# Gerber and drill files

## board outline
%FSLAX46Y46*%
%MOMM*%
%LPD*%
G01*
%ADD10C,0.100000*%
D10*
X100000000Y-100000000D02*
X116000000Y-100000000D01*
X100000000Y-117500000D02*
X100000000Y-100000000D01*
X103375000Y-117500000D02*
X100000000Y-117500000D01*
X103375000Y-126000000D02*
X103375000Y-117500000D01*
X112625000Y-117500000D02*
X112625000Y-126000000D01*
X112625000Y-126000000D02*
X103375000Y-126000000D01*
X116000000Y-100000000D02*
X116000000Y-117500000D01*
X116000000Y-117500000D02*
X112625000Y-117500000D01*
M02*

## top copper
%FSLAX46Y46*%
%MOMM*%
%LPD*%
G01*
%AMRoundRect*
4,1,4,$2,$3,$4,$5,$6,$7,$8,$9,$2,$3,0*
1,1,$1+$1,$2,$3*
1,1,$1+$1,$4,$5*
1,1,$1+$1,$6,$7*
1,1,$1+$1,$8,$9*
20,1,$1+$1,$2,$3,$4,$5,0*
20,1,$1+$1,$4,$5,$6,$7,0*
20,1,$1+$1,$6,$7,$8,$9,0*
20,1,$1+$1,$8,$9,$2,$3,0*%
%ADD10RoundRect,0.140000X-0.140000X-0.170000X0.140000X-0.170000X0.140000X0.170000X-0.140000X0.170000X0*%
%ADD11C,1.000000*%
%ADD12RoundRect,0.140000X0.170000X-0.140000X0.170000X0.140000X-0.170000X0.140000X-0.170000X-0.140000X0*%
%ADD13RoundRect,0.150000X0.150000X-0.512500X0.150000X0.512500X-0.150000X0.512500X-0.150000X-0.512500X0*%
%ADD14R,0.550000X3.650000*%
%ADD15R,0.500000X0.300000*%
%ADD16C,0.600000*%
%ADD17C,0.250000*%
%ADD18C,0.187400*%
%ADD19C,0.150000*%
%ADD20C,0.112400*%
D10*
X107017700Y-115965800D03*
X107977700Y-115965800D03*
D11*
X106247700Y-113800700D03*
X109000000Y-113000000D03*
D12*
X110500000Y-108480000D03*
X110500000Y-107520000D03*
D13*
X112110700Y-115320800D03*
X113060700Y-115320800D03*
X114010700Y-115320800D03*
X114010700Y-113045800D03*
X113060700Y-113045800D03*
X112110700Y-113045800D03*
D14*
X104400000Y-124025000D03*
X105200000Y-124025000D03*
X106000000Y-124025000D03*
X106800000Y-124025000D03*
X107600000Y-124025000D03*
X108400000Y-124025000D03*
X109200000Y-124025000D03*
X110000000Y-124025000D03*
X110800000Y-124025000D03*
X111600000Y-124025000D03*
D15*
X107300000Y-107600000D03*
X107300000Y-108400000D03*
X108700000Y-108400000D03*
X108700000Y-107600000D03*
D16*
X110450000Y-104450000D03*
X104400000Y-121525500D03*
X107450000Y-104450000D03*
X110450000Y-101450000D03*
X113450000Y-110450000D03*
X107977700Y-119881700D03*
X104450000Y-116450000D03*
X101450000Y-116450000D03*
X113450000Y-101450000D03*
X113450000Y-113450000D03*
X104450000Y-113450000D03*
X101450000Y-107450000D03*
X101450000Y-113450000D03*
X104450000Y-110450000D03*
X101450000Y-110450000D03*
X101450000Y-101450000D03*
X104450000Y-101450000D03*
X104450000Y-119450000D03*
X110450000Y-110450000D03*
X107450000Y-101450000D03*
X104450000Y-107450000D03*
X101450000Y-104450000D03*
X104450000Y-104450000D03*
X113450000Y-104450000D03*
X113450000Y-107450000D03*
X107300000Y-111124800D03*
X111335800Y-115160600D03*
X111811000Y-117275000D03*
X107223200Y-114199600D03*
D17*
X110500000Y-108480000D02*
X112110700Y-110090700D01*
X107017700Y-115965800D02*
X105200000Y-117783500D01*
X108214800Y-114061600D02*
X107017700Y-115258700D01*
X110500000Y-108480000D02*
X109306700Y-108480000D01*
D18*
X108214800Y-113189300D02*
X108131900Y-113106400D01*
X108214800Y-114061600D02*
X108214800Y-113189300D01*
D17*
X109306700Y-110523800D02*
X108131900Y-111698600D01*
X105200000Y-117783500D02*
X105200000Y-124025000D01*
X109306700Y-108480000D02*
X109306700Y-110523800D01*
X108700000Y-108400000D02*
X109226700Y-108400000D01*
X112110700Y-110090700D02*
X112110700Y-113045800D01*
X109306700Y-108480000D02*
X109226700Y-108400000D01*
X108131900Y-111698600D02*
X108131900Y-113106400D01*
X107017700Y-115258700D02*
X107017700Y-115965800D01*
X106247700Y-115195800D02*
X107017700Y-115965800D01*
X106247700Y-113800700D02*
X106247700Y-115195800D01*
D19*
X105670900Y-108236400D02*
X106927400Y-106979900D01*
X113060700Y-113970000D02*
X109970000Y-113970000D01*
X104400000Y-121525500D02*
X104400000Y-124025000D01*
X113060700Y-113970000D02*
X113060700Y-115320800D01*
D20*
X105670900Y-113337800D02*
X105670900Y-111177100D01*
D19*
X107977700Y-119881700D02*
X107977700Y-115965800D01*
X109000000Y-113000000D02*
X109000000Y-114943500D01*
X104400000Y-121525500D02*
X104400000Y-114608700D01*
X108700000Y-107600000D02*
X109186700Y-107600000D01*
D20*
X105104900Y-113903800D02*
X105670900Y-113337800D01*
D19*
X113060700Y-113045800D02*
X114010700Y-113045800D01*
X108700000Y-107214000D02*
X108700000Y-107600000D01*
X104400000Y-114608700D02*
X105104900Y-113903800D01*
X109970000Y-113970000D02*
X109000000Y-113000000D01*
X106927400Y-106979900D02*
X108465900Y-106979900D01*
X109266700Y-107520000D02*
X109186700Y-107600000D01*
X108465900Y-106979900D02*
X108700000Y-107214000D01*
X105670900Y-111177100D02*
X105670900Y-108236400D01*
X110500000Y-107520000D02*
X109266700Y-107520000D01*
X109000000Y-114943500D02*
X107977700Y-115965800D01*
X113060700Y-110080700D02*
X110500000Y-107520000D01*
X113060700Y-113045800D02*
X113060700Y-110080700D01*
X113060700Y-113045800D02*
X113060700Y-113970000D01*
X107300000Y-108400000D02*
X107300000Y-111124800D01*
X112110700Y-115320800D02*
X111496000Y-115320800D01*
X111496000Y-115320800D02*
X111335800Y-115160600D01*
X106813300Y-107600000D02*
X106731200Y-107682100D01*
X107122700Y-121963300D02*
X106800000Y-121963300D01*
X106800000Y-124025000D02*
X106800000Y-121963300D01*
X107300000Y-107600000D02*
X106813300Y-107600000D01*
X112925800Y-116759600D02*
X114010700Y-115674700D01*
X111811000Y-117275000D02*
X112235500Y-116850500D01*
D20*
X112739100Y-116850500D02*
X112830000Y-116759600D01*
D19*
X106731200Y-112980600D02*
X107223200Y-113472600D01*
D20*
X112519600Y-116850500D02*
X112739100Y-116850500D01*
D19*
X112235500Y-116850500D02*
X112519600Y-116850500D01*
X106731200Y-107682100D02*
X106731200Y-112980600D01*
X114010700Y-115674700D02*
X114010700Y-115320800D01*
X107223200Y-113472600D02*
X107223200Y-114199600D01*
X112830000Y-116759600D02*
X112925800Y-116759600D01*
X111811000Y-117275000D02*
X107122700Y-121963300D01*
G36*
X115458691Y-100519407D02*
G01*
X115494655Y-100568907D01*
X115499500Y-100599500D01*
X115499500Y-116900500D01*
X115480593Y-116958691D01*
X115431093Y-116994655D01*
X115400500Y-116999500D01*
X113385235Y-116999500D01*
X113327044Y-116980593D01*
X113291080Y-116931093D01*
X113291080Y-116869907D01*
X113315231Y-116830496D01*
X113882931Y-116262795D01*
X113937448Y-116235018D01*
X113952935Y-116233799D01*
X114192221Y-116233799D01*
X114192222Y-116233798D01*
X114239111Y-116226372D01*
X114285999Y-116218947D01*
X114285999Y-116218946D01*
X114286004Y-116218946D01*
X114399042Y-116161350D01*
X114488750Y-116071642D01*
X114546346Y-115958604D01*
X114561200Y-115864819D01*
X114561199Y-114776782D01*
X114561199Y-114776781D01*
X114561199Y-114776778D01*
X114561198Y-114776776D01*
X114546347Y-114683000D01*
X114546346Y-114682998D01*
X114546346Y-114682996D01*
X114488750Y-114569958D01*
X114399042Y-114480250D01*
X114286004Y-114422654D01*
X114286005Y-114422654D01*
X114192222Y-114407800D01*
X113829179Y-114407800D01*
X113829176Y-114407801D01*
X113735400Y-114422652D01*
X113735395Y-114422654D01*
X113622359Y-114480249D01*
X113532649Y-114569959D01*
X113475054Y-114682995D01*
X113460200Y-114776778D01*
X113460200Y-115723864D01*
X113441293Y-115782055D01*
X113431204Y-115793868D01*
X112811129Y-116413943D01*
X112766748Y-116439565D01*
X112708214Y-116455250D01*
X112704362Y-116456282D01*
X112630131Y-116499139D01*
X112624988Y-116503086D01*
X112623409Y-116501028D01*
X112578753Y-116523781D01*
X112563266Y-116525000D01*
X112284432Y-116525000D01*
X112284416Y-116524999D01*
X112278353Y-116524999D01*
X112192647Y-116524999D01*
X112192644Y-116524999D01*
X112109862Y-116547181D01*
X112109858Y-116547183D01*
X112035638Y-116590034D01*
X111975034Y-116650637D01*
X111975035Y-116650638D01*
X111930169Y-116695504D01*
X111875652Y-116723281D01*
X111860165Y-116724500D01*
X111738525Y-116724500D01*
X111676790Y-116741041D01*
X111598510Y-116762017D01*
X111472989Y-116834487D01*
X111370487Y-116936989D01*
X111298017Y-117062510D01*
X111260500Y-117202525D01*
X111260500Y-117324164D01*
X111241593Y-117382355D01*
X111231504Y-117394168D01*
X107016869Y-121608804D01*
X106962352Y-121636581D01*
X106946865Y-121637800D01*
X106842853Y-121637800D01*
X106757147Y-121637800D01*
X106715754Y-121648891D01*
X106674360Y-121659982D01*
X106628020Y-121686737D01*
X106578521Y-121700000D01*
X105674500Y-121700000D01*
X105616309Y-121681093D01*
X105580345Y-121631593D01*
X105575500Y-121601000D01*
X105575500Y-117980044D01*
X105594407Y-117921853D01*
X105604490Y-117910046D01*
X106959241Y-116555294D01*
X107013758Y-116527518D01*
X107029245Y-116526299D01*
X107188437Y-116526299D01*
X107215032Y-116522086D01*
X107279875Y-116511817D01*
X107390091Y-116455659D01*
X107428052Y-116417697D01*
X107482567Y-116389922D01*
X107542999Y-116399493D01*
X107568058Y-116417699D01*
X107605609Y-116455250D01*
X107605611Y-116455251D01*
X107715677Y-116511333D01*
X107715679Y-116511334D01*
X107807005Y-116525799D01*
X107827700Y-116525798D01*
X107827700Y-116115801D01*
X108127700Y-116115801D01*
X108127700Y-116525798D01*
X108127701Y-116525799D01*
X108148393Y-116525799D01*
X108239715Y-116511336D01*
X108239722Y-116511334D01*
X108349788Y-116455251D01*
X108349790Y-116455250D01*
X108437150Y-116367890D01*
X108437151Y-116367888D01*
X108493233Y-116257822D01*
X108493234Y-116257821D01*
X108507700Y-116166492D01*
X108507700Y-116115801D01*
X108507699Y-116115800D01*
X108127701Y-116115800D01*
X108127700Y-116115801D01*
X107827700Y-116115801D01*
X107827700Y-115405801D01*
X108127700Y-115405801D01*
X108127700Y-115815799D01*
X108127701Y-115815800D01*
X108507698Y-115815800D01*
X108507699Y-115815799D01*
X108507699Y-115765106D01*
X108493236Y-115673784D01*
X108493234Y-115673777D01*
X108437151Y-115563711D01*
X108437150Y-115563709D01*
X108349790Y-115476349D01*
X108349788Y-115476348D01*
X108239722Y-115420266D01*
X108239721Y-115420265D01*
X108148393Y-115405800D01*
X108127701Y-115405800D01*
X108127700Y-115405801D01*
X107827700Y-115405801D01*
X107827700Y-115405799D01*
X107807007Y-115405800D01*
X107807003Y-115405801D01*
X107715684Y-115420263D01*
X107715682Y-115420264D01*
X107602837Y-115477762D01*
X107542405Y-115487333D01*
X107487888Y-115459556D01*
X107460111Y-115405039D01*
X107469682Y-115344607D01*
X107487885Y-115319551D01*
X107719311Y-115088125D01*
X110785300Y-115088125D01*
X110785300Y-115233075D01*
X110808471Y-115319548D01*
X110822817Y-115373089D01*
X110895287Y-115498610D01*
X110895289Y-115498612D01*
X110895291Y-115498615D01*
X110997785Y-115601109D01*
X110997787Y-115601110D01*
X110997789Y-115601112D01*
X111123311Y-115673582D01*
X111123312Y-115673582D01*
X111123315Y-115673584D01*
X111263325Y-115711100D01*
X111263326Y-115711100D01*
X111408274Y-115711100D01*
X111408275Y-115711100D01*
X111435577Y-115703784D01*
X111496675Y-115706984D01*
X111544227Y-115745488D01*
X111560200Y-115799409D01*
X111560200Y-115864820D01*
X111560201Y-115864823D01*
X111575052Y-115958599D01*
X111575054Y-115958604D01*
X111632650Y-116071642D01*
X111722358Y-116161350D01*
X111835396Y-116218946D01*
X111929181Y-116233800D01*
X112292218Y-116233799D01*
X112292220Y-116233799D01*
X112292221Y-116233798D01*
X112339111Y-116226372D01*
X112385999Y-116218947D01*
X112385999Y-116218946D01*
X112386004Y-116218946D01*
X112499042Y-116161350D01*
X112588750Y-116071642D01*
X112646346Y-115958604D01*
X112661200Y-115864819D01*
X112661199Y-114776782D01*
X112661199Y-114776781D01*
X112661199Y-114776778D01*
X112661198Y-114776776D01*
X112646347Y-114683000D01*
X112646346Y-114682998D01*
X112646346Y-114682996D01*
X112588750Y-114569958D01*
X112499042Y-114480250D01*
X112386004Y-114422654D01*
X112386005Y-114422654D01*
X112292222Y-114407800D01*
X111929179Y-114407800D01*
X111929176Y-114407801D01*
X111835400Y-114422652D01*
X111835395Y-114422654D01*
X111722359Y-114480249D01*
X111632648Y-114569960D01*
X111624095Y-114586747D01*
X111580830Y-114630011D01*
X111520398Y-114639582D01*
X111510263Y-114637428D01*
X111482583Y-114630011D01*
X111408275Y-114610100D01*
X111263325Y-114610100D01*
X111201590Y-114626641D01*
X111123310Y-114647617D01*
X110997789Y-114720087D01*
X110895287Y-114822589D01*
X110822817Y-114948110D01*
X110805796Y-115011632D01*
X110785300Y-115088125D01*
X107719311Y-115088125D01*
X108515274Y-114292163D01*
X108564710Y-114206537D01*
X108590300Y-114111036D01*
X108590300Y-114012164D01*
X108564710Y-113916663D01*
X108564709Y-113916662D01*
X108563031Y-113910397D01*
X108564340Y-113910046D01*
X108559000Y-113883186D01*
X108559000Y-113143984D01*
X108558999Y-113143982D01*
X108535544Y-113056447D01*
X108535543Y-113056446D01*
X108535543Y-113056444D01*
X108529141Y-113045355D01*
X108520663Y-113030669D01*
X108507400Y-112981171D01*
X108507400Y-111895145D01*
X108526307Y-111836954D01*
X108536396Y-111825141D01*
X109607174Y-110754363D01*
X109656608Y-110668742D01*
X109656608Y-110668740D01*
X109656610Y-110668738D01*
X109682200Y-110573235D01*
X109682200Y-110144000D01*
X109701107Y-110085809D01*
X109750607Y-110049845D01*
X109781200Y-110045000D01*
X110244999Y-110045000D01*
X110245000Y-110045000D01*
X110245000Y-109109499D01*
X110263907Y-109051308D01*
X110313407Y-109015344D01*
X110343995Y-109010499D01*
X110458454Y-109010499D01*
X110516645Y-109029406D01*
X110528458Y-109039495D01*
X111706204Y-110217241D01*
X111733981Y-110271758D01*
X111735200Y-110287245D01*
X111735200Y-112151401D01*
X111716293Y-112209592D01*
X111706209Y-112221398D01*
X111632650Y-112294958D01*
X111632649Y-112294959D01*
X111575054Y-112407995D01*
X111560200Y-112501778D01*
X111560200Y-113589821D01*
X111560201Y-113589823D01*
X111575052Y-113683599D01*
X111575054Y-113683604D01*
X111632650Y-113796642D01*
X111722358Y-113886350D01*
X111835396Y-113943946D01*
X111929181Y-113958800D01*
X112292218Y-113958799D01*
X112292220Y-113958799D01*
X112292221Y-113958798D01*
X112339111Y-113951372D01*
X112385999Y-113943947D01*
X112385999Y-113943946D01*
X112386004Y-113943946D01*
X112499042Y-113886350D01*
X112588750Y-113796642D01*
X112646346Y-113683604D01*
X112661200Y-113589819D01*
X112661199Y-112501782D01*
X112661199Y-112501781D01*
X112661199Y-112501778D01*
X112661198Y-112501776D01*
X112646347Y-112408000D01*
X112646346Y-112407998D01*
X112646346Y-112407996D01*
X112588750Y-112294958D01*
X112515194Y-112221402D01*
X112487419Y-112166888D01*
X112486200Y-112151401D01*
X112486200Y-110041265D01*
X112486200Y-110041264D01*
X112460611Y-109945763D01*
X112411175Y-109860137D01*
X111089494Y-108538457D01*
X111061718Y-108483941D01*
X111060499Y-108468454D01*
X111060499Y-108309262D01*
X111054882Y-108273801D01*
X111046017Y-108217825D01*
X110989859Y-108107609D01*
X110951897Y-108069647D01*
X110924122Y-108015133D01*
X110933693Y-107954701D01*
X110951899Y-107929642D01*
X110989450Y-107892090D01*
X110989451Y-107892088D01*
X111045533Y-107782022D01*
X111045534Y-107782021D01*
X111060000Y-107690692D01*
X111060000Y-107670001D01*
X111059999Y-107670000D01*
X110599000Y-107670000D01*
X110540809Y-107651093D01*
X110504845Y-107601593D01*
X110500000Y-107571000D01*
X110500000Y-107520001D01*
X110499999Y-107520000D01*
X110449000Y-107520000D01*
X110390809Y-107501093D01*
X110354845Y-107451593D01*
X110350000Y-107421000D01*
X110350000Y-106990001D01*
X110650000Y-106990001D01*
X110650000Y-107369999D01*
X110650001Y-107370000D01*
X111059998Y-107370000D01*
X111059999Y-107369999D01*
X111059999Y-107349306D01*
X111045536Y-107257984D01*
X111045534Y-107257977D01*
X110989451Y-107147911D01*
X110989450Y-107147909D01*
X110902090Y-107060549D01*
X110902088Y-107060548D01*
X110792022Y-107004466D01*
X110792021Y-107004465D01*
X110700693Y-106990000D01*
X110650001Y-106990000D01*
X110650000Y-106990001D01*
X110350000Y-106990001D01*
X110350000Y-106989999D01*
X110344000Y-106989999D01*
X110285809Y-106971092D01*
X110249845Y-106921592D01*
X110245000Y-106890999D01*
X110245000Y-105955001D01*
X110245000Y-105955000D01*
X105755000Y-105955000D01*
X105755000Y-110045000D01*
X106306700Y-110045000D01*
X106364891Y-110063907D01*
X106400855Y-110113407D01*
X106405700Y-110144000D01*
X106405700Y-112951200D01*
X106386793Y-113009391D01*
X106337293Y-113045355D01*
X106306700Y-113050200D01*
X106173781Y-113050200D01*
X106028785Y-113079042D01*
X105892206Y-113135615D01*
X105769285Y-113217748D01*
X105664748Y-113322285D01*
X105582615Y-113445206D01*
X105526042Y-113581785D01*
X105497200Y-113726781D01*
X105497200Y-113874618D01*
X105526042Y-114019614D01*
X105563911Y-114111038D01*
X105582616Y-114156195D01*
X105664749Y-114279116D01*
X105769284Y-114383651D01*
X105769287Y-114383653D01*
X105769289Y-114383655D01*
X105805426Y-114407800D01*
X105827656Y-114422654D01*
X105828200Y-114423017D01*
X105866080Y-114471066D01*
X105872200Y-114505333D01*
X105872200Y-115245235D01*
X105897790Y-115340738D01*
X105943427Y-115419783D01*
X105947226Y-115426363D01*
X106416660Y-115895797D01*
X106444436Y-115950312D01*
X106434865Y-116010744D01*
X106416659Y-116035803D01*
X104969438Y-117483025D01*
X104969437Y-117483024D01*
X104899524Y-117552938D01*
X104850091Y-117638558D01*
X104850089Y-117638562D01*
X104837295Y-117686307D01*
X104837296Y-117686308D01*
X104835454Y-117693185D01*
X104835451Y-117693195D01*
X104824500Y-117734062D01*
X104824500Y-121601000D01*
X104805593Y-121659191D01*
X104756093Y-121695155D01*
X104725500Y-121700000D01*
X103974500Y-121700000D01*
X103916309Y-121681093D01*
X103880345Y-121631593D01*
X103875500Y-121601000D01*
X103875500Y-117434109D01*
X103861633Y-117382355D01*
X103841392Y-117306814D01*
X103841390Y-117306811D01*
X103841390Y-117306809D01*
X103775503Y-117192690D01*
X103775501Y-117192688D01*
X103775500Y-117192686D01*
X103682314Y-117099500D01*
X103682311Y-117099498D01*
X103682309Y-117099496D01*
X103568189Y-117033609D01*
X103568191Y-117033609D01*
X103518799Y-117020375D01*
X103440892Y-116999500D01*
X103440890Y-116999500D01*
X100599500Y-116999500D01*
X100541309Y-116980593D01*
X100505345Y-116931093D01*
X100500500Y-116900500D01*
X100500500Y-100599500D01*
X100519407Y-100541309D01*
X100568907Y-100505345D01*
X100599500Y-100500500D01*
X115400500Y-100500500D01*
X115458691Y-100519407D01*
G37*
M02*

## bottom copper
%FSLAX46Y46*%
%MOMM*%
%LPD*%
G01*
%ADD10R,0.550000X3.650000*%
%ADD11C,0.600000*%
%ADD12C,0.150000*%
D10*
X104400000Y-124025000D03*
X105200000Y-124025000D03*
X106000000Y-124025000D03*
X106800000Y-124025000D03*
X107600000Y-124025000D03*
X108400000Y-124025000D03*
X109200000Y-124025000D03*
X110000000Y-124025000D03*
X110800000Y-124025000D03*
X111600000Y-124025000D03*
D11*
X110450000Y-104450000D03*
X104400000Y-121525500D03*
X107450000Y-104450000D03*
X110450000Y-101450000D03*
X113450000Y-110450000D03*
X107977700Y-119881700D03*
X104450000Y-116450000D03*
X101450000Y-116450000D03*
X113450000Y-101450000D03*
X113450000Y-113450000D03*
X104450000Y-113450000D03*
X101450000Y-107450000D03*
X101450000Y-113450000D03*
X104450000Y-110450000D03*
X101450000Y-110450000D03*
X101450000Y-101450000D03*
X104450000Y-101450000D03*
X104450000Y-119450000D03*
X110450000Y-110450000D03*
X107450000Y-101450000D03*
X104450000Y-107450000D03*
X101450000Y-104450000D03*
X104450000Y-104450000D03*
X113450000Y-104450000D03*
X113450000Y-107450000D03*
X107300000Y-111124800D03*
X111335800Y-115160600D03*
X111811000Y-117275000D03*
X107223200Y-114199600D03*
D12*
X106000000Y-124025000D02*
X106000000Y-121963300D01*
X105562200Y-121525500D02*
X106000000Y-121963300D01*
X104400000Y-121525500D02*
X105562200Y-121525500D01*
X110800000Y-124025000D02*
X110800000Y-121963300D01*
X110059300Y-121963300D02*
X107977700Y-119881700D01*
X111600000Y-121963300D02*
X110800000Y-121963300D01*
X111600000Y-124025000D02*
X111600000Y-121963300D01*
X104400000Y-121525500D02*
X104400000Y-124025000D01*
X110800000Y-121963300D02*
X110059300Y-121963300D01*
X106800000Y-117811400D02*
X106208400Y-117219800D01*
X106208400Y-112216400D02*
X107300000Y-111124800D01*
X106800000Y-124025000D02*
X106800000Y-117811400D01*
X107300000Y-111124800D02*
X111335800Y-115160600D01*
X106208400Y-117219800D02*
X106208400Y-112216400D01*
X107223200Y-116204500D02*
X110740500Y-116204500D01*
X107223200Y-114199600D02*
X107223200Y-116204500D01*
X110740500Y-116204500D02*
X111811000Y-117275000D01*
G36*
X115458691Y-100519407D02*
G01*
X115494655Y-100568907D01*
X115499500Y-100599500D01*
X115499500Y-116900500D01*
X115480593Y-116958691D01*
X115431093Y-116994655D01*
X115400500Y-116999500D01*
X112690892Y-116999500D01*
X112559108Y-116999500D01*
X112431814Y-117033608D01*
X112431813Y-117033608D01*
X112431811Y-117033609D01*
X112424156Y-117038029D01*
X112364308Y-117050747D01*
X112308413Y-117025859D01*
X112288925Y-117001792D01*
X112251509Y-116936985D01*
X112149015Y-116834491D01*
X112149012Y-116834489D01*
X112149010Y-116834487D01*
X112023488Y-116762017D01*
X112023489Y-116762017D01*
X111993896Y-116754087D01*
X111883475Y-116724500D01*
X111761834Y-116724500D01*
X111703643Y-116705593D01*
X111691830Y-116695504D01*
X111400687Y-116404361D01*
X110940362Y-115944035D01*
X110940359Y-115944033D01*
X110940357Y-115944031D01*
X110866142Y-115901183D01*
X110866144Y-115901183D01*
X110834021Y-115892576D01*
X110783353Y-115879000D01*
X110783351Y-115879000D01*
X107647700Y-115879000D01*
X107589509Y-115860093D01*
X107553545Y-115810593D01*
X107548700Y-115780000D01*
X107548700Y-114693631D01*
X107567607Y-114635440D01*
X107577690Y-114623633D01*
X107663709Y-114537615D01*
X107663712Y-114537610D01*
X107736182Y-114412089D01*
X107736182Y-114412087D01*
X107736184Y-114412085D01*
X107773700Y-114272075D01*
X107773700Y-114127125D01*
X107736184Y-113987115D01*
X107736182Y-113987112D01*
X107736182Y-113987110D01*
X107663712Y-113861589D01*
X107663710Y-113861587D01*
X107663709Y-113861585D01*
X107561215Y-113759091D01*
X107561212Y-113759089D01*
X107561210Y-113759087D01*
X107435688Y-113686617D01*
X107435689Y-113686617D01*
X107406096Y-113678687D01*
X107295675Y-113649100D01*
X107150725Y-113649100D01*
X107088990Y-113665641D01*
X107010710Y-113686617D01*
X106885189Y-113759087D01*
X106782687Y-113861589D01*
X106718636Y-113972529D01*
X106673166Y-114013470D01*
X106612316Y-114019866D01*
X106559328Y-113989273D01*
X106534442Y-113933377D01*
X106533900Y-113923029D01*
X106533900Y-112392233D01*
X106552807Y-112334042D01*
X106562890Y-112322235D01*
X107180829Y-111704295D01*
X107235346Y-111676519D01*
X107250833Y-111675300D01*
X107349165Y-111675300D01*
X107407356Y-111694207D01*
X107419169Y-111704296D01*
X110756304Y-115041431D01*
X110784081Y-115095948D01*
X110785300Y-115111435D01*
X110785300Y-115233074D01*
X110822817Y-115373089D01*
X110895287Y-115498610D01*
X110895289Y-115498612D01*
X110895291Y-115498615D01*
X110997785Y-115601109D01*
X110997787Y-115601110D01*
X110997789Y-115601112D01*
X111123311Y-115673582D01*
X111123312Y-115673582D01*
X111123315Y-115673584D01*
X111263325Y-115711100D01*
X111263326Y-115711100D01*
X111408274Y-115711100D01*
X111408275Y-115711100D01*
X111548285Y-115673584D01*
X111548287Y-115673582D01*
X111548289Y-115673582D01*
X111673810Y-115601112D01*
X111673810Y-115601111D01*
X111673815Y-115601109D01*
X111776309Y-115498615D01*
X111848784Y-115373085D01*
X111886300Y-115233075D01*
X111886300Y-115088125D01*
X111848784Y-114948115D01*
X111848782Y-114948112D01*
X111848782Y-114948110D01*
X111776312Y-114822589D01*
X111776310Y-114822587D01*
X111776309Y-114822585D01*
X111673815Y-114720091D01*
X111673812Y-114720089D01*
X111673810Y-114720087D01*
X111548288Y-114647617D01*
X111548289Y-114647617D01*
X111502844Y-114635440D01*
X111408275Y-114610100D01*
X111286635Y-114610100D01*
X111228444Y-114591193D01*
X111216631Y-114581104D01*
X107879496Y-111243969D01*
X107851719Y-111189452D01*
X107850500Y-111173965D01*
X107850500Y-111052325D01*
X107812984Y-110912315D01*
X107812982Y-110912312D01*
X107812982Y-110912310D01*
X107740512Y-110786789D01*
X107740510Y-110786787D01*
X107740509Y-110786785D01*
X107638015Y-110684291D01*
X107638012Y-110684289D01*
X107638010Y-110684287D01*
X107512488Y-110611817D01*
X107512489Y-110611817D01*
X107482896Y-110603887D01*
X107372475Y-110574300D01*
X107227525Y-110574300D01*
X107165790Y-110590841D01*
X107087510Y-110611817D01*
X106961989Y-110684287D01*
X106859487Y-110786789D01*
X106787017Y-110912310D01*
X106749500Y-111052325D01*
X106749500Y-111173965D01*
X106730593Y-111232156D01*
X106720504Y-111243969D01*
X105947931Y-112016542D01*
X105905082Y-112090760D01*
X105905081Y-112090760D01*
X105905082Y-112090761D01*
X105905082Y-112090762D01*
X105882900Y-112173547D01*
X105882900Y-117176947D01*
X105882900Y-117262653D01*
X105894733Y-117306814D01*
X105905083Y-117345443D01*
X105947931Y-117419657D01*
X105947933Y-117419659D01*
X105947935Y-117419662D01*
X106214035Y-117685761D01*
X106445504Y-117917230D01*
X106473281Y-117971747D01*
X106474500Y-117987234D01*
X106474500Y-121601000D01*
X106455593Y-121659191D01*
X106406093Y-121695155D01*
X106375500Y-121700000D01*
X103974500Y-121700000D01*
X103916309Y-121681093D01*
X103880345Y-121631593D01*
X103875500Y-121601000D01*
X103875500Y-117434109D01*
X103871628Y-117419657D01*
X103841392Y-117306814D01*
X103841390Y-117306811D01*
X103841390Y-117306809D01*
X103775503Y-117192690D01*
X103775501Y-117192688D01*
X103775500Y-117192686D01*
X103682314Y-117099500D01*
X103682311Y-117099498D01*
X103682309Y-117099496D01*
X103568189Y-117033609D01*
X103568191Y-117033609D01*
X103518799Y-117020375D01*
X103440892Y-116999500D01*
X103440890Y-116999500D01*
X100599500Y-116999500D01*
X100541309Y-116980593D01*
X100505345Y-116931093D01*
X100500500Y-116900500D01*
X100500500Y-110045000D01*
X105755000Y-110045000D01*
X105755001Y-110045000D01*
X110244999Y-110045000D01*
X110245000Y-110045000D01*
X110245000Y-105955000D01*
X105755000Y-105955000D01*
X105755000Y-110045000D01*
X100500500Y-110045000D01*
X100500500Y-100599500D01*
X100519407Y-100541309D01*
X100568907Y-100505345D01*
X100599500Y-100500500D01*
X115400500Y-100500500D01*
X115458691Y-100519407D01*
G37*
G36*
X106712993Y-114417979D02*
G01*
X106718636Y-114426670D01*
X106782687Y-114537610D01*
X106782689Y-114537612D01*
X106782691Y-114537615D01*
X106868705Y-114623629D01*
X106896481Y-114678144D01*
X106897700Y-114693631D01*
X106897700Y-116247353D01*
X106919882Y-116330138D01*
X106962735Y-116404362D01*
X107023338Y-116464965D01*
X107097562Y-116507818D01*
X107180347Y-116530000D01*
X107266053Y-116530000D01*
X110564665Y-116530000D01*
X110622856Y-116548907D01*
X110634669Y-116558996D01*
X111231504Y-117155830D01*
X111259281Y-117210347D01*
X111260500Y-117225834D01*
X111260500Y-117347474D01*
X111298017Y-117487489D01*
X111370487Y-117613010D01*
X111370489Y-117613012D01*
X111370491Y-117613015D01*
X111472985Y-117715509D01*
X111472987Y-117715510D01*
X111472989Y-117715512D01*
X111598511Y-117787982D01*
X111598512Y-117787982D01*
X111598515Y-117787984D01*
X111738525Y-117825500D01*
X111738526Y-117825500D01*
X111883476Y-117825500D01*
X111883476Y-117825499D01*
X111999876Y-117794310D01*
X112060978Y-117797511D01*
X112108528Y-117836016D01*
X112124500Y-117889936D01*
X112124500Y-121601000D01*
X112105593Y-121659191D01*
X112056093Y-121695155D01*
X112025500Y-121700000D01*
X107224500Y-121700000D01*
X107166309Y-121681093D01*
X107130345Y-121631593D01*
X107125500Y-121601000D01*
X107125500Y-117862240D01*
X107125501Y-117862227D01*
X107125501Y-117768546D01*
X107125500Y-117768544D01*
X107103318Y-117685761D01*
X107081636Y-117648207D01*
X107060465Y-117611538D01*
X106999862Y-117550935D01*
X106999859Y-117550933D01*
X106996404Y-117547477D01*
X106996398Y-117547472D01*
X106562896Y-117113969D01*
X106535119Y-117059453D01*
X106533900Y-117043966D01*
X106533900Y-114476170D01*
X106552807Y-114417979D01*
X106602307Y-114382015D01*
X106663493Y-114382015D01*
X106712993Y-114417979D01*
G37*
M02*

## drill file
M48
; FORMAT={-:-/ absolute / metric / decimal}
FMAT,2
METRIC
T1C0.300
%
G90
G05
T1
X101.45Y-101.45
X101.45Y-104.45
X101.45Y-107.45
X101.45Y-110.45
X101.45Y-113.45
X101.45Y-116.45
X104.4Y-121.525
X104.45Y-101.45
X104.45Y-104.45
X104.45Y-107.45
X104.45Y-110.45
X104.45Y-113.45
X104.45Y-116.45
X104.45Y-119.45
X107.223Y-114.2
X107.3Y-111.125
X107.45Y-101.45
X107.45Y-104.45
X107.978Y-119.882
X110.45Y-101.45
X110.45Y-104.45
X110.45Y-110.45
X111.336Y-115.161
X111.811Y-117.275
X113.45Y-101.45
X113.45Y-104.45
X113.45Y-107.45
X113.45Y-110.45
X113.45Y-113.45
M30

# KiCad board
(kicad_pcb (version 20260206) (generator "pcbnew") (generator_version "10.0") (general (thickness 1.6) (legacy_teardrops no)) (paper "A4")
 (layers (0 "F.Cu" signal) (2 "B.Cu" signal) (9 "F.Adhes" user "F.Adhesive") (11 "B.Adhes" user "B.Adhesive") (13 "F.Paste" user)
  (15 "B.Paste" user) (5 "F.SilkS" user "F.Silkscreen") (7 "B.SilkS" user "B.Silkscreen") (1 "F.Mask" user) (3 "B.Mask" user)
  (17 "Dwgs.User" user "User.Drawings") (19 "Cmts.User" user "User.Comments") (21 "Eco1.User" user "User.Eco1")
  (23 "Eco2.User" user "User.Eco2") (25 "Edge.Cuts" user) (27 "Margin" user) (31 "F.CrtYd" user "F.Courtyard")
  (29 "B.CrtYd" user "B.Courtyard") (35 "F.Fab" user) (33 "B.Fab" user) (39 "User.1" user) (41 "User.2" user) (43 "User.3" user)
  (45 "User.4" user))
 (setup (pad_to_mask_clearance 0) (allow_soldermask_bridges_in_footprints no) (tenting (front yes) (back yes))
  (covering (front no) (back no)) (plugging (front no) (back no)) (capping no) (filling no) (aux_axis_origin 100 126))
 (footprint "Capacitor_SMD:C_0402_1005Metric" (layer "F.Cu") (at 107.4977 115.9658)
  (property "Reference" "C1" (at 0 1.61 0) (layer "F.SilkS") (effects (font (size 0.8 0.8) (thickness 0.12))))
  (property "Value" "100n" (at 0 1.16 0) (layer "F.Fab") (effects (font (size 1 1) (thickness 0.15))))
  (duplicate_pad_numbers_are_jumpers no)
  (pad "1" smd roundrect (at -0.48 0) (size 0.56 0.62) (layers "F.Cu" "F.Mask" "F.Paste") (roundrect_rratio 0.25) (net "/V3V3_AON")
   (zone_connect 1))
  (pad "2" smd roundrect (at 0.48 0) (size 0.56 0.62) (layers "F.Cu" "F.Mask" "F.Paste") (roundrect_rratio 0.25) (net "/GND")
   (zone_connect 1)))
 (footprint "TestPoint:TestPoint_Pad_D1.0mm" (layer "F.Cu") (at 106.2477 113.8007)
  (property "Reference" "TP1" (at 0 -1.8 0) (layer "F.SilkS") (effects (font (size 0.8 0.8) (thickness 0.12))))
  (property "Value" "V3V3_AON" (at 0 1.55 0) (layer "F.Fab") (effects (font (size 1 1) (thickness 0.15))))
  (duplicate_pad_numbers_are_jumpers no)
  (pad "1" smd circle (at 0 0) (size 1 1) (layers "F.Cu" "F.Mask") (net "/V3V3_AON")))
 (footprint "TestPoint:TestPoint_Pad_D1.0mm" (layer "F.Cu") (at 109 113)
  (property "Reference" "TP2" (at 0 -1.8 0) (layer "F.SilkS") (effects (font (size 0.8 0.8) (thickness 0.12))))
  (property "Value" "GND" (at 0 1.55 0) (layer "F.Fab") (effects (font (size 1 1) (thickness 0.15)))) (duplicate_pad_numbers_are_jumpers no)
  (pad "1" smd circle (at 0 0) (size 1 1) (layers "F.Cu" "F.Mask") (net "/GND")))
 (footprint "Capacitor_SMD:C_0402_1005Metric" (layer "F.Cu") (at 110.5 108 90)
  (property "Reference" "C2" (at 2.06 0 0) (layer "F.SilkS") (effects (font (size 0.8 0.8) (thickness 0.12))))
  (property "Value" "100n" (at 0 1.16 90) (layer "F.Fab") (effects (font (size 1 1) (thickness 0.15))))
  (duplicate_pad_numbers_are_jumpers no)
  (pad "1" smd roundrect (at -0.48 0 90) (size 0.56 0.62) (layers "F.Cu" "F.Mask" "F.Paste") (roundrect_rratio 0.25) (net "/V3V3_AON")
   (zone_connect 1))
  (pad "2" smd roundrect (at 0.48 0 90) (size 0.56 0.62) (layers "F.Cu" "F.Mask" "F.Paste") (roundrect_rratio 0.25) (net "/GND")
   (zone_connect 1)))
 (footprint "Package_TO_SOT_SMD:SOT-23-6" (layer "F.Cu") (at 113.0607 114.1833 90)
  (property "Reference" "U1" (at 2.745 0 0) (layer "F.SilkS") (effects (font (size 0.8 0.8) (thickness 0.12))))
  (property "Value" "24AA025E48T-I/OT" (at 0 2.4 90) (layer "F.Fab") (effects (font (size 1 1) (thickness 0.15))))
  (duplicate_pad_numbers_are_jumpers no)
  (pad "1" smd roundrect (at -1.1375 -0.95 90) (size 1.325 0.6) (layers "F.Cu" "F.Mask" "F.Paste") (roundrect_rratio 0.25) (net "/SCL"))
  (pad "2" smd roundrect (at -1.1375 0 90) (size 1.325 0.6) (layers "F.Cu" "F.Mask" "F.Paste") (roundrect_rratio 0.25) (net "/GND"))
  (pad "3" smd roundrect (at -1.1375 0.95 90) (size 1.325 0.6) (layers "F.Cu" "F.Mask" "F.Paste") (roundrect_rratio 0.25) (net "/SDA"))
  (pad "4" smd roundrect (at 1.1375 0.95 90) (size 1.325 0.6) (layers "F.Cu" "F.Mask" "F.Paste") (roundrect_rratio 0.25) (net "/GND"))
  (pad "5" smd roundrect (at 1.1375 0 90) (size 1.325 0.6) (layers "F.Cu" "F.Mask" "F.Paste") (roundrect_rratio 0.25) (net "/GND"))
  (pad "6" smd roundrect (at 1.1375 -0.95 90) (size 1.325 0.6) (layers "F.Cu" "F.Mask" "F.Paste") (roundrect_rratio 0.25) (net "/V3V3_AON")))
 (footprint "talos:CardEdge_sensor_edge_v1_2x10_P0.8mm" (layer "F.Cu") (at 108 124.35)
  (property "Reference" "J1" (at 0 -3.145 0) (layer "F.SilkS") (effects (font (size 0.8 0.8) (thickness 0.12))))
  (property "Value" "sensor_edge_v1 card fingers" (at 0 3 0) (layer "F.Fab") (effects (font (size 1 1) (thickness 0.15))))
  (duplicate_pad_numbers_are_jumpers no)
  (pad "1" smd rect (at -3.6 -0.325) (size 0.55 3.65) (layers "F.Cu" "F.Mask") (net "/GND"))
  (pad "2" smd rect (at -3.6 -0.325) (size 0.55 3.65) (layers "B.Cu" "B.Mask") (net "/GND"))
  (pad "3" smd rect (at -2.8 -0.325) (size 0.55 3.65) (layers "F.Cu" "F.Mask") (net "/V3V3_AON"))
  (pad "4" smd rect (at -2.8 -0.325) (size 0.55 3.65) (layers "B.Cu" "B.Mask") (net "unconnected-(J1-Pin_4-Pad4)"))
  (pad "5" smd rect (at -2 -0.325) (size 0.55 3.65) (layers "F.Cu" "F.Mask") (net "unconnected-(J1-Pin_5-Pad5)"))
  (pad "6" smd rect (at -2 -0.325) (size 0.55 3.65) (layers "B.Cu" "B.Mask") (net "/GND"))
  (pad "7" smd rect (at -1.2 -0.325) (size 0.55 3.65) (layers "F.Cu" "F.Mask") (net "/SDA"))
  (pad "8" smd rect (at -1.2 -0.325) (size 0.55 3.65) (layers "B.Cu" "B.Mask") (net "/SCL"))
  (pad "9" smd rect (at -0.4 -0.325) (size 0.55 3.65) (layers "F.Cu" "F.Mask") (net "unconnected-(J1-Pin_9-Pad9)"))
  (pad "10" smd rect (at -0.4 -0.325) (size 0.55 3.65) (layers "B.Cu" "B.Mask") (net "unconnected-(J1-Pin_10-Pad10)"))
  (pad "11" smd rect (at 0.4 -0.325) (size 0.55 3.65) (layers "F.Cu" "F.Mask") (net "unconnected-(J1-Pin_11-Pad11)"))
  (pad "12" smd rect (at 0.4 -0.325) (size 0.55 3.65) (layers "B.Cu" "B.Mask") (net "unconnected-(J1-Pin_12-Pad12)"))
  (pad "13" smd rect (at 1.2 -0.325) (size 0.55 3.65) (layers "F.Cu" "F.Mask") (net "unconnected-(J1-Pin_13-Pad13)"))
  (pad "14" smd rect (at 1.2 -0.325) (size 0.55 3.65) (layers "B.Cu" "B.Mask") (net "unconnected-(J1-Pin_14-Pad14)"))
  (pad "15" smd rect (at 2 -0.325) (size 0.55 3.65) (layers "F.Cu" "F.Mask") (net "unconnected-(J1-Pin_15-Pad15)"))
  (pad "16" smd rect (at 2 -0.325) (size 0.55 3.65) (layers "B.Cu" "B.Mask") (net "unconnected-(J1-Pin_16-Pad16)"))
  (pad "17" smd rect (at 2.8 -0.325) (size 0.55 3.65) (layers "F.Cu" "F.Mask") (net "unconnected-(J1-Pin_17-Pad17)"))
  (pad "18" smd rect (at 2.8 -0.325) (size 0.55 3.65) (layers "B.Cu" "B.Mask") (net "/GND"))
  (pad "19" smd rect (at 3.6 -0.325) (size 0.55 3.65) (layers "F.Cu" "F.Mask") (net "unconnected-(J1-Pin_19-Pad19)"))
  (pad "20" smd rect (at 3.6 -0.325) (size 0.55 3.65) (layers "B.Cu" "B.Mask") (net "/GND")))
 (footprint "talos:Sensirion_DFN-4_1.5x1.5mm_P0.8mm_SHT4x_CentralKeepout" (layer "F.Cu") (at 108 108)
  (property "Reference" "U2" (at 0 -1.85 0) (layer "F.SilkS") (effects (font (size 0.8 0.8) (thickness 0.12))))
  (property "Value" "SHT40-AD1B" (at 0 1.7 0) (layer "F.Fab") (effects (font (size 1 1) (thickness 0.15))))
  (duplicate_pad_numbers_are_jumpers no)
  (pad "1" smd rect (at -0.7 -0.4) (size 0.5 0.3) (layers "F.Cu" "F.Mask" "F.Paste") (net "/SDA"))
  (pad "2" smd rect (at -0.7 0.4) (size 0.5 0.3) (layers "F.Cu" "F.Mask" "F.Paste") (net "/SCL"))
  (pad "3" smd rect (at 0.7 0.4) (size 0.5 0.3) (layers "F.Cu" "F.Mask" "F.Paste") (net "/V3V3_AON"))
  (pad "4" smd rect (at 0.7 -0.4) (size 0.5 0.3) (layers "F.Cu" "F.Mask" "F.Paste") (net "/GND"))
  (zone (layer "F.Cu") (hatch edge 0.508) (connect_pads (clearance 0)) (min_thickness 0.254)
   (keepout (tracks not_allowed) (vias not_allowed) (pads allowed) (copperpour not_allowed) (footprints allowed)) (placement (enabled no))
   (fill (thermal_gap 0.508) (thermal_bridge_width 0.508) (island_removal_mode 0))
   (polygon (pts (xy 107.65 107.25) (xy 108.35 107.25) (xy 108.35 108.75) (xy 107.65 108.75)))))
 (gr_line (start 100 100) (end 116 100) (stroke (width 0.1) (type default)) (layer "Edge.Cuts"))
 (gr_line (start 100 117.5) (end 100 100) (stroke (width 0.1) (type default)) (layer "Edge.Cuts"))
 (gr_line (start 103.375 117.5) (end 100 117.5) (stroke (width 0.1) (type default)) (layer "Edge.Cuts"))
 (gr_line (start 103.375 126) (end 103.375 117.5) (stroke (width 0.1) (type default)) (layer "Edge.Cuts"))
 (gr_line (start 112.625 117.5) (end 112.625 126) (stroke (width 0.1) (type default)) (layer "Edge.Cuts"))
 (gr_line (start 112.625 126) (end 103.375 126) (stroke (width 0.1) (type default)) (layer "Edge.Cuts"))
 (gr_line (start 116 100) (end 116 117.5) (stroke (width 0.1) (type default)) (layer "Edge.Cuts"))
 (gr_line (start 116 117.5) (end 112.625 117.5) (stroke (width 0.1) (type default)) (layer "Edge.Cuts"))
 (segment (start 110.5 108.48) (end 112.1107 110.0907) (width 0.25) (layer "F.Cu") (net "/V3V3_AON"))
 (segment (start 107.0177 115.9658) (end 105.2 117.7835) (width 0.25) (layer "F.Cu") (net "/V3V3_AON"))
 (segment (start 108.2148 114.0616) (end 107.0177 115.2587) (width 0.25) (layer "F.Cu") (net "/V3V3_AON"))
 (segment (start 110.5 108.48) (end 109.3067 108.48) (width 0.25) (layer "F.Cu") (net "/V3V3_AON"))
 (segment (start 108.2148 113.1893) (end 108.1319 113.1064) (width 0.1874) (layer "F.Cu") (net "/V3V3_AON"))
 (segment (start 108.2148 114.0616) (end 108.2148 113.1893) (width 0.1874) (layer "F.Cu") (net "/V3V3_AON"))
 (segment (start 109.3067 110.5238) (end 108.1319 111.6986) (width 0.25) (layer "F.Cu") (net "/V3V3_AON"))
 (segment (start 105.2 117.7835) (end 105.2 124.025) (width 0.25) (layer "F.Cu") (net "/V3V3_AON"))
 (segment (start 109.3067 108.48) (end 109.3067 110.5238) (width 0.25) (layer "F.Cu") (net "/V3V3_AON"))
 (segment (start 108.7 108.4) (end 109.2267 108.4) (width 0.25) (layer "F.Cu") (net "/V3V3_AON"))
 (segment (start 112.1107 110.0907) (end 112.1107 113.0458) (width 0.25) (layer "F.Cu") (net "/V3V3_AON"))
 (segment (start 109.3067 108.48) (end 109.2267 108.4) (width 0.25) (layer "F.Cu") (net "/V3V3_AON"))
 (segment (start 108.1319 111.6986) (end 108.1319 113.1064) (width 0.25) (layer "F.Cu") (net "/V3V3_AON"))
 (segment (start 107.0177 115.2587) (end 107.0177 115.9658) (width 0.25) (layer "F.Cu") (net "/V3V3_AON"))
 (segment (start 106.2477 115.1958) (end 107.0177 115.9658) (width 0.25) (layer "F.Cu") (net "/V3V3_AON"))
 (segment (start 106.2477 113.8007) (end 106.2477 115.1958) (width 0.25) (layer "F.Cu") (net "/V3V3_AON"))
 (segment (start 105.6709 108.2364) (end 106.9274 106.9799) (width 0.15) (layer "F.Cu") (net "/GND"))
 (segment (start 113.0607 113.97) (end 109.97 113.97) (width 0.15) (layer "F.Cu") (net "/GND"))
 (segment (start 104.4 121.5255) (end 104.4 124.025) (width 0.15) (layer "F.Cu") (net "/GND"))
 (segment (start 113.0607 113.97) (end 113.0607 115.3208) (width 0.15) (layer "F.Cu") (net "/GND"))
 (segment (start 105.6709 113.3378) (end 105.6709 111.1771) (width 0.1124) (layer "F.Cu") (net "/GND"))
 (segment (start 107.9777 119.8817) (end 107.9777 115.9658) (width 0.15) (layer "F.Cu") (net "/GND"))
 (segment (start 109 113) (end 109 114.9435) (width 0.15) (layer "F.Cu") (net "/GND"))
 (segment (start 104.4 121.5255) (end 104.4 114.6087) (width 0.15) (layer "F.Cu") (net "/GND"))
 (segment (start 108.7 107.6) (end 109.1867 107.6) (width 0.15) (layer "F.Cu") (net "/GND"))
 (segment (start 105.1049 113.9038) (end 105.6709 113.3378) (width 0.1124) (layer "F.Cu") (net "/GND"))
 (segment (start 113.0607 113.0458) (end 114.0107 113.0458) (width 0.15) (layer "F.Cu") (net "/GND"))
 (segment (start 108.7 107.214) (end 108.7 107.6) (width 0.15) (layer "F.Cu") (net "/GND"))
 (segment (start 104.4 114.6087) (end 105.1049 113.9038) (width 0.15) (layer "F.Cu") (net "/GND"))
 (segment (start 109.97 113.97) (end 109 113) (width 0.15) (layer "F.Cu") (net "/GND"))
 (segment (start 106.9274 106.9799) (end 108.4659 106.9799) (width 0.15) (layer "F.Cu") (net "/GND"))
 (segment (start 109.2667 107.52) (end 109.1867 107.6) (width 0.15) (layer "F.Cu") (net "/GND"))
 (segment (start 108.4659 106.9799) (end 108.7 107.214) (width 0.15) (layer "F.Cu") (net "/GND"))
 (segment (start 105.6709 111.1771) (end 105.6709 108.2364) (width 0.15) (layer "F.Cu") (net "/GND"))
 (segment (start 110.5 107.52) (end 109.2667 107.52) (width 0.15) (layer "F.Cu") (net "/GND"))
 (segment (start 109 114.9435) (end 107.9777 115.9658) (width 0.15) (layer "F.Cu") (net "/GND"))
 (segment (start 113.0607 110.0807) (end 110.5 107.52) (width 0.15) (layer "F.Cu") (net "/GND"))
 (segment (start 113.0607 113.0458) (end 113.0607 110.0807) (width 0.15) (layer "F.Cu") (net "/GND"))
 (segment (start 113.0607 113.0458) (end 113.0607 113.97) (width 0.15) (layer "F.Cu") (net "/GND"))
 (via (at 110.45 104.45) (size 0.6) (drill 0.3) (layers "F.Cu" "B.Cu") (locked yes) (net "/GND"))
 (via (at 104.4 121.5255) (size 0.6) (drill 0.3) (layers "F.Cu" "B.Cu") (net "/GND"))
 (via (at 107.45 104.45) (size 0.6) (drill 0.3) (layers "F.Cu" "B.Cu") (locked yes) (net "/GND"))
 (via (at 110.45 101.45) (size 0.6) (drill 0.3) (layers "F.Cu" "B.Cu") (locked yes) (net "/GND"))
 (via (at 113.45 110.45) (size 0.6) (drill 0.3) (layers "F.Cu" "B.Cu") (locked yes) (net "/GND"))
 (via (at 107.9777 119.8817) (size 0.6) (drill 0.3) (layers "F.Cu" "B.Cu") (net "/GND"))
 (via (at 104.45 116.45) (size 0.6) (drill 0.3) (layers "F.Cu" "B.Cu") (locked yes) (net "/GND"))
 (via (at 101.45 116.45) (size 0.6) (drill 0.3) (layers "F.Cu" "B.Cu") (locked yes) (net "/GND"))
 (via (at 113.45 101.45) (size 0.6) (drill 0.3) (layers "F.Cu" "B.Cu") (locked yes) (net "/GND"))
 (via (at 113.45 113.45) (size 0.6) (drill 0.3) (layers "F.Cu" "B.Cu") (locked yes) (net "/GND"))
 (via (at 104.45 113.45) (size 0.6) (drill 0.3) (layers "F.Cu" "B.Cu") (locked yes) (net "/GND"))
 (via (at 101.45 107.45) (size 0.6) (drill 0.3) (layers "F.Cu" "B.Cu") (locked yes) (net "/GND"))
 (via (at 101.45 113.45) (size 0.6) (drill 0.3) (layers "F.Cu" "B.Cu") (locked yes) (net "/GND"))
 (via (at 104.45 110.45) (size 0.6) (drill 0.3) (layers "F.Cu" "B.Cu") (locked yes) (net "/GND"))
 (via (at 101.45 110.45) (size 0.6) (drill 0.3) (layers "F.Cu" "B.Cu") (locked yes) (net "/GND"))
 (via (at 101.45 101.45) (size 0.6) (drill 0.3) (layers "F.Cu" "B.Cu") (locked yes) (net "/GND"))
 (via (at 104.45 101.45) (size 0.6) (drill 0.3) (layers "F.Cu" "B.Cu") (locked yes) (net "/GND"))
 (via (at 104.45 119.45) (size 0.6) (drill 0.3) (layers "F.Cu" "B.Cu") (locked yes) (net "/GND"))
 (via (at 110.45 110.45) (size 0.6) (drill 0.3) (layers "F.Cu" "B.Cu") (locked yes) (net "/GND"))
 (via (at 107.45 101.45) (size 0.6) (drill 0.3) (layers "F.Cu" "B.Cu") (locked yes) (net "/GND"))
 (via (at 104.45 107.45) (size 0.6) (drill 0.3) (layers "F.Cu" "B.Cu") (locked yes) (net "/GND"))
 (via (at 101.45 104.45) (size 0.6) (drill 0.3) (layers "F.Cu" "B.Cu") (locked yes) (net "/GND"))
 (via (at 104.45 104.45) (size 0.6) (drill 0.3) (layers "F.Cu" "B.Cu") (locked yes) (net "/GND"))
 (via (at 113.45 104.45) (size 0.6) (drill 0.3) (layers "F.Cu" "B.Cu") (locked yes) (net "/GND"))
 (via (at 113.45 107.45) (size 0.6) (drill 0.3) (layers "F.Cu" "B.Cu") (locked yes) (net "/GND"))
 (segment (start 106 124.025) (end 106 121.9633) (width 0.15) (layer "B.Cu") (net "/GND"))
 (segment (start 105.5622 121.5255) (end 106 121.9633) (width 0.15) (layer "B.Cu") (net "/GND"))
 (segment (start 104.4 121.5255) (end 105.5622 121.5255) (width 0.15) (layer "B.Cu") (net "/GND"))
 (segment (start 110.8 124.025) (end 110.8 121.9633) (width 0.15) (layer "B.Cu") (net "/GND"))
 (segment (start 110.0593 121.9633) (end 107.9777 119.8817) (width 0.15) (layer "B.Cu") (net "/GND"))
 (segment (start 111.6 121.9633) (end 110.8 121.9633) (width 0.15) (layer "B.Cu") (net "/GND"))
 (segment (start 111.6 124.025) (end 111.6 121.9633) (width 0.15) (layer "B.Cu") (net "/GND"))
 (segment (start 104.4 121.5255) (end 104.4 124.025) (width 0.15) (layer "B.Cu") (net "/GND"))
 (segment (start 110.8 121.9633) (end 110.0593 121.9633) (width 0.15) (layer "B.Cu") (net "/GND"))
 (segment (start 107.3 108.4) (end 107.3 111.1248) (width 0.15) (layer "F.Cu") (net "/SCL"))
 (segment (start 112.1107 115.3208) (end 111.496 115.3208) (width 0.15) (layer "F.Cu") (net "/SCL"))
 (segment (start 111.496 115.3208) (end 111.3358 115.1606) (width 0.15) (layer "F.Cu") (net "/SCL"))
 (via (at 107.3 111.1248) (size 0.6) (drill 0.3) (layers "F.Cu" "B.Cu") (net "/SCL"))
 (via (at 111.3358 115.1606) (size 0.6) (drill 0.3) (layers "F.Cu" "B.Cu") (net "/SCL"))
 (segment (start 106.8 117.8114) (end 106.2084 117.2198) (width 0.15) (layer "B.Cu") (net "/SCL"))
 (segment (start 106.2084 112.2164) (end 107.3 111.1248) (width 0.15) (layer "B.Cu") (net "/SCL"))
 (segment (start 106.8 124.025) (end 106.8 117.8114) (width 0.15) (layer "B.Cu") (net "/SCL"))
 (segment (start 107.3 111.1248) (end 111.3358 115.1606) (width 0.15) (layer "B.Cu") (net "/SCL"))
 (segment (start 106.2084 117.2198) (end 106.2084 112.2164) (width 0.15) (layer "B.Cu") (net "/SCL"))
 (segment (start 106.8133 107.6) (end 106.7312 107.6821) (width 0.15) (layer "F.Cu") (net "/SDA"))
 (segment (start 107.1227 121.9633) (end 106.8 121.9633) (width 0.15) (layer "F.Cu") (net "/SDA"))
 (segment (start 106.8 124.025) (end 106.8 121.9633) (width 0.15) (layer "F.Cu") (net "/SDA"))
 (segment (start 107.3 107.6) (end 106.8133 107.6) (width 0.15) (layer "F.Cu") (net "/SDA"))
 (segment (start 112.9258 116.7596) (end 114.0107 115.6747) (width 0.15) (layer "F.Cu") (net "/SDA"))
 (segment (start 111.811 117.275) (end 112.2355 116.8505) (width 0.15) (layer "F.Cu") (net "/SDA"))
 (segment (start 112.7391 116.8505) (end 112.83 116.7596) (width 0.1124) (layer "F.Cu") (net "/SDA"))
 (segment (start 106.7312 112.9806) (end 107.2232 113.4726) (width 0.15) (layer "F.Cu") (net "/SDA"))
 (segment (start 112.5196 116.8505) (end 112.7391 116.8505) (width 0.1124) (layer "F.Cu") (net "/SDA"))
 (segment (start 112.2355 116.8505) (end 112.5196 116.8505) (width 0.15) (layer "F.Cu") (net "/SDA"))
 (segment (start 106.7312 107.6821) (end 106.7312 112.9806) (width 0.15) (layer "F.Cu") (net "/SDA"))
 (segment (start 114.0107 115.6747) (end 114.0107 115.3208) (width 0.15) (layer "F.Cu") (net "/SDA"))
 (segment (start 107.2232 113.4726) (end 107.2232 114.1996) (width 0.15) (layer "F.Cu") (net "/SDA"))
 (segment (start 112.83 116.7596) (end 112.9258 116.7596) (width 0.15) (layer "F.Cu") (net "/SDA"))
 (segment (start 111.811 117.275) (end 107.1227 121.9633) (width 0.15) (layer "F.Cu") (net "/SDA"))
 (via (at 111.811 117.275) (size 0.6) (drill 0.3) (layers "F.Cu" "B.Cu") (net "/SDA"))
 (via (at 107.2232 114.1996) (size 0.6) (drill 0.3) (layers "F.Cu" "B.Cu") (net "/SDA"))
 (segment (start 107.2232 116.2045) (end 110.7405 116.2045) (width 0.15) (layer "B.Cu") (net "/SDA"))
 (segment (start 107.2232 114.1996) (end 107.2232 116.2045) (width 0.15) (layer "B.Cu") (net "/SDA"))
 (segment (start 110.7405 116.2045) (end 111.811 117.275) (width 0.15) (layer "B.Cu") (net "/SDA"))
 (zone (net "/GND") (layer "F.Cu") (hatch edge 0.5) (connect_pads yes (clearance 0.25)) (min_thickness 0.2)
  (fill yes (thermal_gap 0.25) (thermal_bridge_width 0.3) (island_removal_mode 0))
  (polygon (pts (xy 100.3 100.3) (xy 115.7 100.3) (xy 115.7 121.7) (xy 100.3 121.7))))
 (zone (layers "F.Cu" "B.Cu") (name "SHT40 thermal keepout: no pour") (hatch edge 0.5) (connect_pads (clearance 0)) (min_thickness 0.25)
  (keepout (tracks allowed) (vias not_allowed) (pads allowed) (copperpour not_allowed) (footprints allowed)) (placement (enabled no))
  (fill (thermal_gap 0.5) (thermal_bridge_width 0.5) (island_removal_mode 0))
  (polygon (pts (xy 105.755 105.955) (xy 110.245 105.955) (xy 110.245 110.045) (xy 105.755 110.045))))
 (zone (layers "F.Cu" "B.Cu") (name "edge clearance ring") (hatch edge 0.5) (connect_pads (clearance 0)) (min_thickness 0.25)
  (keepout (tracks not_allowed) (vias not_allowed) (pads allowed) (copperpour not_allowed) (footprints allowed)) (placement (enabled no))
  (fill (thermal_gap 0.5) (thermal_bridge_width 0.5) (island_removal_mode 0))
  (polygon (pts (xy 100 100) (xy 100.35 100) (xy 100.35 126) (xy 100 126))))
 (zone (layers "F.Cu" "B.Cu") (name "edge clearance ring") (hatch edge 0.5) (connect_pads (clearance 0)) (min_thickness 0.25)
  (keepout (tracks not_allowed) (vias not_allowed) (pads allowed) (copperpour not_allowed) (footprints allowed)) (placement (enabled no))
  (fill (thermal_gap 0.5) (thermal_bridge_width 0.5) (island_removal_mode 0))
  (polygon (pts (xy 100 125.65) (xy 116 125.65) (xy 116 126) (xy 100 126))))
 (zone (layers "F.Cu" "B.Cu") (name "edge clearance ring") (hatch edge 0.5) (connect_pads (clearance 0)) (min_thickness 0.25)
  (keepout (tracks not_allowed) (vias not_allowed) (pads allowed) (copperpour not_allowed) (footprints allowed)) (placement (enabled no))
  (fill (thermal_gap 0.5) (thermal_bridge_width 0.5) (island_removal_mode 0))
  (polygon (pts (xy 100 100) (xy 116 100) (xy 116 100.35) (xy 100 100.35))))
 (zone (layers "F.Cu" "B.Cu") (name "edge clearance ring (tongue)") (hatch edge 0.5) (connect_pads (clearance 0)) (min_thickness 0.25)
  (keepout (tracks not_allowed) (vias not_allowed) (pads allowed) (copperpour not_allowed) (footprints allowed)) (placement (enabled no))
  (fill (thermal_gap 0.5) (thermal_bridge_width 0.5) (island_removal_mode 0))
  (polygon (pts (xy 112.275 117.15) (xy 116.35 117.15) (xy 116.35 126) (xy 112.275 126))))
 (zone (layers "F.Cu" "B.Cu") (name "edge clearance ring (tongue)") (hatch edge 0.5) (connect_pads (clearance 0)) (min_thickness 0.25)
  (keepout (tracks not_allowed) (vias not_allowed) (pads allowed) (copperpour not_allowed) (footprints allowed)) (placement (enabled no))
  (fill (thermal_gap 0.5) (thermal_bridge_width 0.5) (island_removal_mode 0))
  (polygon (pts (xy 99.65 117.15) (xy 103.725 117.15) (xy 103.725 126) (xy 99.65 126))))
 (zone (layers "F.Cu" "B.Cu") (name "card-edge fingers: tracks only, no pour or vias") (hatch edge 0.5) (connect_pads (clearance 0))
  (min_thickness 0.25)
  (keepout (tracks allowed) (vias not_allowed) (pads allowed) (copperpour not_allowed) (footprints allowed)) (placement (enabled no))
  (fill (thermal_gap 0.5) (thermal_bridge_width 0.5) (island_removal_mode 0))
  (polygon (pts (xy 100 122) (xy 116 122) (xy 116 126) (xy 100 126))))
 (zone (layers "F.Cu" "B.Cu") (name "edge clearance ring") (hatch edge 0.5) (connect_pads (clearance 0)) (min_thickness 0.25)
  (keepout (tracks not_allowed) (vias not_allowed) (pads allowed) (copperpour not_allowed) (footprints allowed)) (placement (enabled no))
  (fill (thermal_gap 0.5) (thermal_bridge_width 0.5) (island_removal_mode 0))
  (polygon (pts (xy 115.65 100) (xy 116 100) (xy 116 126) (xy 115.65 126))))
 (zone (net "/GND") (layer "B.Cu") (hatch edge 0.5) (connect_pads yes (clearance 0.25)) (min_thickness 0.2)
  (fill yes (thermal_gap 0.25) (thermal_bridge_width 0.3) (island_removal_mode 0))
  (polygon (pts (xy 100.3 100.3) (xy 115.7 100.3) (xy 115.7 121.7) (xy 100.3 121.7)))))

